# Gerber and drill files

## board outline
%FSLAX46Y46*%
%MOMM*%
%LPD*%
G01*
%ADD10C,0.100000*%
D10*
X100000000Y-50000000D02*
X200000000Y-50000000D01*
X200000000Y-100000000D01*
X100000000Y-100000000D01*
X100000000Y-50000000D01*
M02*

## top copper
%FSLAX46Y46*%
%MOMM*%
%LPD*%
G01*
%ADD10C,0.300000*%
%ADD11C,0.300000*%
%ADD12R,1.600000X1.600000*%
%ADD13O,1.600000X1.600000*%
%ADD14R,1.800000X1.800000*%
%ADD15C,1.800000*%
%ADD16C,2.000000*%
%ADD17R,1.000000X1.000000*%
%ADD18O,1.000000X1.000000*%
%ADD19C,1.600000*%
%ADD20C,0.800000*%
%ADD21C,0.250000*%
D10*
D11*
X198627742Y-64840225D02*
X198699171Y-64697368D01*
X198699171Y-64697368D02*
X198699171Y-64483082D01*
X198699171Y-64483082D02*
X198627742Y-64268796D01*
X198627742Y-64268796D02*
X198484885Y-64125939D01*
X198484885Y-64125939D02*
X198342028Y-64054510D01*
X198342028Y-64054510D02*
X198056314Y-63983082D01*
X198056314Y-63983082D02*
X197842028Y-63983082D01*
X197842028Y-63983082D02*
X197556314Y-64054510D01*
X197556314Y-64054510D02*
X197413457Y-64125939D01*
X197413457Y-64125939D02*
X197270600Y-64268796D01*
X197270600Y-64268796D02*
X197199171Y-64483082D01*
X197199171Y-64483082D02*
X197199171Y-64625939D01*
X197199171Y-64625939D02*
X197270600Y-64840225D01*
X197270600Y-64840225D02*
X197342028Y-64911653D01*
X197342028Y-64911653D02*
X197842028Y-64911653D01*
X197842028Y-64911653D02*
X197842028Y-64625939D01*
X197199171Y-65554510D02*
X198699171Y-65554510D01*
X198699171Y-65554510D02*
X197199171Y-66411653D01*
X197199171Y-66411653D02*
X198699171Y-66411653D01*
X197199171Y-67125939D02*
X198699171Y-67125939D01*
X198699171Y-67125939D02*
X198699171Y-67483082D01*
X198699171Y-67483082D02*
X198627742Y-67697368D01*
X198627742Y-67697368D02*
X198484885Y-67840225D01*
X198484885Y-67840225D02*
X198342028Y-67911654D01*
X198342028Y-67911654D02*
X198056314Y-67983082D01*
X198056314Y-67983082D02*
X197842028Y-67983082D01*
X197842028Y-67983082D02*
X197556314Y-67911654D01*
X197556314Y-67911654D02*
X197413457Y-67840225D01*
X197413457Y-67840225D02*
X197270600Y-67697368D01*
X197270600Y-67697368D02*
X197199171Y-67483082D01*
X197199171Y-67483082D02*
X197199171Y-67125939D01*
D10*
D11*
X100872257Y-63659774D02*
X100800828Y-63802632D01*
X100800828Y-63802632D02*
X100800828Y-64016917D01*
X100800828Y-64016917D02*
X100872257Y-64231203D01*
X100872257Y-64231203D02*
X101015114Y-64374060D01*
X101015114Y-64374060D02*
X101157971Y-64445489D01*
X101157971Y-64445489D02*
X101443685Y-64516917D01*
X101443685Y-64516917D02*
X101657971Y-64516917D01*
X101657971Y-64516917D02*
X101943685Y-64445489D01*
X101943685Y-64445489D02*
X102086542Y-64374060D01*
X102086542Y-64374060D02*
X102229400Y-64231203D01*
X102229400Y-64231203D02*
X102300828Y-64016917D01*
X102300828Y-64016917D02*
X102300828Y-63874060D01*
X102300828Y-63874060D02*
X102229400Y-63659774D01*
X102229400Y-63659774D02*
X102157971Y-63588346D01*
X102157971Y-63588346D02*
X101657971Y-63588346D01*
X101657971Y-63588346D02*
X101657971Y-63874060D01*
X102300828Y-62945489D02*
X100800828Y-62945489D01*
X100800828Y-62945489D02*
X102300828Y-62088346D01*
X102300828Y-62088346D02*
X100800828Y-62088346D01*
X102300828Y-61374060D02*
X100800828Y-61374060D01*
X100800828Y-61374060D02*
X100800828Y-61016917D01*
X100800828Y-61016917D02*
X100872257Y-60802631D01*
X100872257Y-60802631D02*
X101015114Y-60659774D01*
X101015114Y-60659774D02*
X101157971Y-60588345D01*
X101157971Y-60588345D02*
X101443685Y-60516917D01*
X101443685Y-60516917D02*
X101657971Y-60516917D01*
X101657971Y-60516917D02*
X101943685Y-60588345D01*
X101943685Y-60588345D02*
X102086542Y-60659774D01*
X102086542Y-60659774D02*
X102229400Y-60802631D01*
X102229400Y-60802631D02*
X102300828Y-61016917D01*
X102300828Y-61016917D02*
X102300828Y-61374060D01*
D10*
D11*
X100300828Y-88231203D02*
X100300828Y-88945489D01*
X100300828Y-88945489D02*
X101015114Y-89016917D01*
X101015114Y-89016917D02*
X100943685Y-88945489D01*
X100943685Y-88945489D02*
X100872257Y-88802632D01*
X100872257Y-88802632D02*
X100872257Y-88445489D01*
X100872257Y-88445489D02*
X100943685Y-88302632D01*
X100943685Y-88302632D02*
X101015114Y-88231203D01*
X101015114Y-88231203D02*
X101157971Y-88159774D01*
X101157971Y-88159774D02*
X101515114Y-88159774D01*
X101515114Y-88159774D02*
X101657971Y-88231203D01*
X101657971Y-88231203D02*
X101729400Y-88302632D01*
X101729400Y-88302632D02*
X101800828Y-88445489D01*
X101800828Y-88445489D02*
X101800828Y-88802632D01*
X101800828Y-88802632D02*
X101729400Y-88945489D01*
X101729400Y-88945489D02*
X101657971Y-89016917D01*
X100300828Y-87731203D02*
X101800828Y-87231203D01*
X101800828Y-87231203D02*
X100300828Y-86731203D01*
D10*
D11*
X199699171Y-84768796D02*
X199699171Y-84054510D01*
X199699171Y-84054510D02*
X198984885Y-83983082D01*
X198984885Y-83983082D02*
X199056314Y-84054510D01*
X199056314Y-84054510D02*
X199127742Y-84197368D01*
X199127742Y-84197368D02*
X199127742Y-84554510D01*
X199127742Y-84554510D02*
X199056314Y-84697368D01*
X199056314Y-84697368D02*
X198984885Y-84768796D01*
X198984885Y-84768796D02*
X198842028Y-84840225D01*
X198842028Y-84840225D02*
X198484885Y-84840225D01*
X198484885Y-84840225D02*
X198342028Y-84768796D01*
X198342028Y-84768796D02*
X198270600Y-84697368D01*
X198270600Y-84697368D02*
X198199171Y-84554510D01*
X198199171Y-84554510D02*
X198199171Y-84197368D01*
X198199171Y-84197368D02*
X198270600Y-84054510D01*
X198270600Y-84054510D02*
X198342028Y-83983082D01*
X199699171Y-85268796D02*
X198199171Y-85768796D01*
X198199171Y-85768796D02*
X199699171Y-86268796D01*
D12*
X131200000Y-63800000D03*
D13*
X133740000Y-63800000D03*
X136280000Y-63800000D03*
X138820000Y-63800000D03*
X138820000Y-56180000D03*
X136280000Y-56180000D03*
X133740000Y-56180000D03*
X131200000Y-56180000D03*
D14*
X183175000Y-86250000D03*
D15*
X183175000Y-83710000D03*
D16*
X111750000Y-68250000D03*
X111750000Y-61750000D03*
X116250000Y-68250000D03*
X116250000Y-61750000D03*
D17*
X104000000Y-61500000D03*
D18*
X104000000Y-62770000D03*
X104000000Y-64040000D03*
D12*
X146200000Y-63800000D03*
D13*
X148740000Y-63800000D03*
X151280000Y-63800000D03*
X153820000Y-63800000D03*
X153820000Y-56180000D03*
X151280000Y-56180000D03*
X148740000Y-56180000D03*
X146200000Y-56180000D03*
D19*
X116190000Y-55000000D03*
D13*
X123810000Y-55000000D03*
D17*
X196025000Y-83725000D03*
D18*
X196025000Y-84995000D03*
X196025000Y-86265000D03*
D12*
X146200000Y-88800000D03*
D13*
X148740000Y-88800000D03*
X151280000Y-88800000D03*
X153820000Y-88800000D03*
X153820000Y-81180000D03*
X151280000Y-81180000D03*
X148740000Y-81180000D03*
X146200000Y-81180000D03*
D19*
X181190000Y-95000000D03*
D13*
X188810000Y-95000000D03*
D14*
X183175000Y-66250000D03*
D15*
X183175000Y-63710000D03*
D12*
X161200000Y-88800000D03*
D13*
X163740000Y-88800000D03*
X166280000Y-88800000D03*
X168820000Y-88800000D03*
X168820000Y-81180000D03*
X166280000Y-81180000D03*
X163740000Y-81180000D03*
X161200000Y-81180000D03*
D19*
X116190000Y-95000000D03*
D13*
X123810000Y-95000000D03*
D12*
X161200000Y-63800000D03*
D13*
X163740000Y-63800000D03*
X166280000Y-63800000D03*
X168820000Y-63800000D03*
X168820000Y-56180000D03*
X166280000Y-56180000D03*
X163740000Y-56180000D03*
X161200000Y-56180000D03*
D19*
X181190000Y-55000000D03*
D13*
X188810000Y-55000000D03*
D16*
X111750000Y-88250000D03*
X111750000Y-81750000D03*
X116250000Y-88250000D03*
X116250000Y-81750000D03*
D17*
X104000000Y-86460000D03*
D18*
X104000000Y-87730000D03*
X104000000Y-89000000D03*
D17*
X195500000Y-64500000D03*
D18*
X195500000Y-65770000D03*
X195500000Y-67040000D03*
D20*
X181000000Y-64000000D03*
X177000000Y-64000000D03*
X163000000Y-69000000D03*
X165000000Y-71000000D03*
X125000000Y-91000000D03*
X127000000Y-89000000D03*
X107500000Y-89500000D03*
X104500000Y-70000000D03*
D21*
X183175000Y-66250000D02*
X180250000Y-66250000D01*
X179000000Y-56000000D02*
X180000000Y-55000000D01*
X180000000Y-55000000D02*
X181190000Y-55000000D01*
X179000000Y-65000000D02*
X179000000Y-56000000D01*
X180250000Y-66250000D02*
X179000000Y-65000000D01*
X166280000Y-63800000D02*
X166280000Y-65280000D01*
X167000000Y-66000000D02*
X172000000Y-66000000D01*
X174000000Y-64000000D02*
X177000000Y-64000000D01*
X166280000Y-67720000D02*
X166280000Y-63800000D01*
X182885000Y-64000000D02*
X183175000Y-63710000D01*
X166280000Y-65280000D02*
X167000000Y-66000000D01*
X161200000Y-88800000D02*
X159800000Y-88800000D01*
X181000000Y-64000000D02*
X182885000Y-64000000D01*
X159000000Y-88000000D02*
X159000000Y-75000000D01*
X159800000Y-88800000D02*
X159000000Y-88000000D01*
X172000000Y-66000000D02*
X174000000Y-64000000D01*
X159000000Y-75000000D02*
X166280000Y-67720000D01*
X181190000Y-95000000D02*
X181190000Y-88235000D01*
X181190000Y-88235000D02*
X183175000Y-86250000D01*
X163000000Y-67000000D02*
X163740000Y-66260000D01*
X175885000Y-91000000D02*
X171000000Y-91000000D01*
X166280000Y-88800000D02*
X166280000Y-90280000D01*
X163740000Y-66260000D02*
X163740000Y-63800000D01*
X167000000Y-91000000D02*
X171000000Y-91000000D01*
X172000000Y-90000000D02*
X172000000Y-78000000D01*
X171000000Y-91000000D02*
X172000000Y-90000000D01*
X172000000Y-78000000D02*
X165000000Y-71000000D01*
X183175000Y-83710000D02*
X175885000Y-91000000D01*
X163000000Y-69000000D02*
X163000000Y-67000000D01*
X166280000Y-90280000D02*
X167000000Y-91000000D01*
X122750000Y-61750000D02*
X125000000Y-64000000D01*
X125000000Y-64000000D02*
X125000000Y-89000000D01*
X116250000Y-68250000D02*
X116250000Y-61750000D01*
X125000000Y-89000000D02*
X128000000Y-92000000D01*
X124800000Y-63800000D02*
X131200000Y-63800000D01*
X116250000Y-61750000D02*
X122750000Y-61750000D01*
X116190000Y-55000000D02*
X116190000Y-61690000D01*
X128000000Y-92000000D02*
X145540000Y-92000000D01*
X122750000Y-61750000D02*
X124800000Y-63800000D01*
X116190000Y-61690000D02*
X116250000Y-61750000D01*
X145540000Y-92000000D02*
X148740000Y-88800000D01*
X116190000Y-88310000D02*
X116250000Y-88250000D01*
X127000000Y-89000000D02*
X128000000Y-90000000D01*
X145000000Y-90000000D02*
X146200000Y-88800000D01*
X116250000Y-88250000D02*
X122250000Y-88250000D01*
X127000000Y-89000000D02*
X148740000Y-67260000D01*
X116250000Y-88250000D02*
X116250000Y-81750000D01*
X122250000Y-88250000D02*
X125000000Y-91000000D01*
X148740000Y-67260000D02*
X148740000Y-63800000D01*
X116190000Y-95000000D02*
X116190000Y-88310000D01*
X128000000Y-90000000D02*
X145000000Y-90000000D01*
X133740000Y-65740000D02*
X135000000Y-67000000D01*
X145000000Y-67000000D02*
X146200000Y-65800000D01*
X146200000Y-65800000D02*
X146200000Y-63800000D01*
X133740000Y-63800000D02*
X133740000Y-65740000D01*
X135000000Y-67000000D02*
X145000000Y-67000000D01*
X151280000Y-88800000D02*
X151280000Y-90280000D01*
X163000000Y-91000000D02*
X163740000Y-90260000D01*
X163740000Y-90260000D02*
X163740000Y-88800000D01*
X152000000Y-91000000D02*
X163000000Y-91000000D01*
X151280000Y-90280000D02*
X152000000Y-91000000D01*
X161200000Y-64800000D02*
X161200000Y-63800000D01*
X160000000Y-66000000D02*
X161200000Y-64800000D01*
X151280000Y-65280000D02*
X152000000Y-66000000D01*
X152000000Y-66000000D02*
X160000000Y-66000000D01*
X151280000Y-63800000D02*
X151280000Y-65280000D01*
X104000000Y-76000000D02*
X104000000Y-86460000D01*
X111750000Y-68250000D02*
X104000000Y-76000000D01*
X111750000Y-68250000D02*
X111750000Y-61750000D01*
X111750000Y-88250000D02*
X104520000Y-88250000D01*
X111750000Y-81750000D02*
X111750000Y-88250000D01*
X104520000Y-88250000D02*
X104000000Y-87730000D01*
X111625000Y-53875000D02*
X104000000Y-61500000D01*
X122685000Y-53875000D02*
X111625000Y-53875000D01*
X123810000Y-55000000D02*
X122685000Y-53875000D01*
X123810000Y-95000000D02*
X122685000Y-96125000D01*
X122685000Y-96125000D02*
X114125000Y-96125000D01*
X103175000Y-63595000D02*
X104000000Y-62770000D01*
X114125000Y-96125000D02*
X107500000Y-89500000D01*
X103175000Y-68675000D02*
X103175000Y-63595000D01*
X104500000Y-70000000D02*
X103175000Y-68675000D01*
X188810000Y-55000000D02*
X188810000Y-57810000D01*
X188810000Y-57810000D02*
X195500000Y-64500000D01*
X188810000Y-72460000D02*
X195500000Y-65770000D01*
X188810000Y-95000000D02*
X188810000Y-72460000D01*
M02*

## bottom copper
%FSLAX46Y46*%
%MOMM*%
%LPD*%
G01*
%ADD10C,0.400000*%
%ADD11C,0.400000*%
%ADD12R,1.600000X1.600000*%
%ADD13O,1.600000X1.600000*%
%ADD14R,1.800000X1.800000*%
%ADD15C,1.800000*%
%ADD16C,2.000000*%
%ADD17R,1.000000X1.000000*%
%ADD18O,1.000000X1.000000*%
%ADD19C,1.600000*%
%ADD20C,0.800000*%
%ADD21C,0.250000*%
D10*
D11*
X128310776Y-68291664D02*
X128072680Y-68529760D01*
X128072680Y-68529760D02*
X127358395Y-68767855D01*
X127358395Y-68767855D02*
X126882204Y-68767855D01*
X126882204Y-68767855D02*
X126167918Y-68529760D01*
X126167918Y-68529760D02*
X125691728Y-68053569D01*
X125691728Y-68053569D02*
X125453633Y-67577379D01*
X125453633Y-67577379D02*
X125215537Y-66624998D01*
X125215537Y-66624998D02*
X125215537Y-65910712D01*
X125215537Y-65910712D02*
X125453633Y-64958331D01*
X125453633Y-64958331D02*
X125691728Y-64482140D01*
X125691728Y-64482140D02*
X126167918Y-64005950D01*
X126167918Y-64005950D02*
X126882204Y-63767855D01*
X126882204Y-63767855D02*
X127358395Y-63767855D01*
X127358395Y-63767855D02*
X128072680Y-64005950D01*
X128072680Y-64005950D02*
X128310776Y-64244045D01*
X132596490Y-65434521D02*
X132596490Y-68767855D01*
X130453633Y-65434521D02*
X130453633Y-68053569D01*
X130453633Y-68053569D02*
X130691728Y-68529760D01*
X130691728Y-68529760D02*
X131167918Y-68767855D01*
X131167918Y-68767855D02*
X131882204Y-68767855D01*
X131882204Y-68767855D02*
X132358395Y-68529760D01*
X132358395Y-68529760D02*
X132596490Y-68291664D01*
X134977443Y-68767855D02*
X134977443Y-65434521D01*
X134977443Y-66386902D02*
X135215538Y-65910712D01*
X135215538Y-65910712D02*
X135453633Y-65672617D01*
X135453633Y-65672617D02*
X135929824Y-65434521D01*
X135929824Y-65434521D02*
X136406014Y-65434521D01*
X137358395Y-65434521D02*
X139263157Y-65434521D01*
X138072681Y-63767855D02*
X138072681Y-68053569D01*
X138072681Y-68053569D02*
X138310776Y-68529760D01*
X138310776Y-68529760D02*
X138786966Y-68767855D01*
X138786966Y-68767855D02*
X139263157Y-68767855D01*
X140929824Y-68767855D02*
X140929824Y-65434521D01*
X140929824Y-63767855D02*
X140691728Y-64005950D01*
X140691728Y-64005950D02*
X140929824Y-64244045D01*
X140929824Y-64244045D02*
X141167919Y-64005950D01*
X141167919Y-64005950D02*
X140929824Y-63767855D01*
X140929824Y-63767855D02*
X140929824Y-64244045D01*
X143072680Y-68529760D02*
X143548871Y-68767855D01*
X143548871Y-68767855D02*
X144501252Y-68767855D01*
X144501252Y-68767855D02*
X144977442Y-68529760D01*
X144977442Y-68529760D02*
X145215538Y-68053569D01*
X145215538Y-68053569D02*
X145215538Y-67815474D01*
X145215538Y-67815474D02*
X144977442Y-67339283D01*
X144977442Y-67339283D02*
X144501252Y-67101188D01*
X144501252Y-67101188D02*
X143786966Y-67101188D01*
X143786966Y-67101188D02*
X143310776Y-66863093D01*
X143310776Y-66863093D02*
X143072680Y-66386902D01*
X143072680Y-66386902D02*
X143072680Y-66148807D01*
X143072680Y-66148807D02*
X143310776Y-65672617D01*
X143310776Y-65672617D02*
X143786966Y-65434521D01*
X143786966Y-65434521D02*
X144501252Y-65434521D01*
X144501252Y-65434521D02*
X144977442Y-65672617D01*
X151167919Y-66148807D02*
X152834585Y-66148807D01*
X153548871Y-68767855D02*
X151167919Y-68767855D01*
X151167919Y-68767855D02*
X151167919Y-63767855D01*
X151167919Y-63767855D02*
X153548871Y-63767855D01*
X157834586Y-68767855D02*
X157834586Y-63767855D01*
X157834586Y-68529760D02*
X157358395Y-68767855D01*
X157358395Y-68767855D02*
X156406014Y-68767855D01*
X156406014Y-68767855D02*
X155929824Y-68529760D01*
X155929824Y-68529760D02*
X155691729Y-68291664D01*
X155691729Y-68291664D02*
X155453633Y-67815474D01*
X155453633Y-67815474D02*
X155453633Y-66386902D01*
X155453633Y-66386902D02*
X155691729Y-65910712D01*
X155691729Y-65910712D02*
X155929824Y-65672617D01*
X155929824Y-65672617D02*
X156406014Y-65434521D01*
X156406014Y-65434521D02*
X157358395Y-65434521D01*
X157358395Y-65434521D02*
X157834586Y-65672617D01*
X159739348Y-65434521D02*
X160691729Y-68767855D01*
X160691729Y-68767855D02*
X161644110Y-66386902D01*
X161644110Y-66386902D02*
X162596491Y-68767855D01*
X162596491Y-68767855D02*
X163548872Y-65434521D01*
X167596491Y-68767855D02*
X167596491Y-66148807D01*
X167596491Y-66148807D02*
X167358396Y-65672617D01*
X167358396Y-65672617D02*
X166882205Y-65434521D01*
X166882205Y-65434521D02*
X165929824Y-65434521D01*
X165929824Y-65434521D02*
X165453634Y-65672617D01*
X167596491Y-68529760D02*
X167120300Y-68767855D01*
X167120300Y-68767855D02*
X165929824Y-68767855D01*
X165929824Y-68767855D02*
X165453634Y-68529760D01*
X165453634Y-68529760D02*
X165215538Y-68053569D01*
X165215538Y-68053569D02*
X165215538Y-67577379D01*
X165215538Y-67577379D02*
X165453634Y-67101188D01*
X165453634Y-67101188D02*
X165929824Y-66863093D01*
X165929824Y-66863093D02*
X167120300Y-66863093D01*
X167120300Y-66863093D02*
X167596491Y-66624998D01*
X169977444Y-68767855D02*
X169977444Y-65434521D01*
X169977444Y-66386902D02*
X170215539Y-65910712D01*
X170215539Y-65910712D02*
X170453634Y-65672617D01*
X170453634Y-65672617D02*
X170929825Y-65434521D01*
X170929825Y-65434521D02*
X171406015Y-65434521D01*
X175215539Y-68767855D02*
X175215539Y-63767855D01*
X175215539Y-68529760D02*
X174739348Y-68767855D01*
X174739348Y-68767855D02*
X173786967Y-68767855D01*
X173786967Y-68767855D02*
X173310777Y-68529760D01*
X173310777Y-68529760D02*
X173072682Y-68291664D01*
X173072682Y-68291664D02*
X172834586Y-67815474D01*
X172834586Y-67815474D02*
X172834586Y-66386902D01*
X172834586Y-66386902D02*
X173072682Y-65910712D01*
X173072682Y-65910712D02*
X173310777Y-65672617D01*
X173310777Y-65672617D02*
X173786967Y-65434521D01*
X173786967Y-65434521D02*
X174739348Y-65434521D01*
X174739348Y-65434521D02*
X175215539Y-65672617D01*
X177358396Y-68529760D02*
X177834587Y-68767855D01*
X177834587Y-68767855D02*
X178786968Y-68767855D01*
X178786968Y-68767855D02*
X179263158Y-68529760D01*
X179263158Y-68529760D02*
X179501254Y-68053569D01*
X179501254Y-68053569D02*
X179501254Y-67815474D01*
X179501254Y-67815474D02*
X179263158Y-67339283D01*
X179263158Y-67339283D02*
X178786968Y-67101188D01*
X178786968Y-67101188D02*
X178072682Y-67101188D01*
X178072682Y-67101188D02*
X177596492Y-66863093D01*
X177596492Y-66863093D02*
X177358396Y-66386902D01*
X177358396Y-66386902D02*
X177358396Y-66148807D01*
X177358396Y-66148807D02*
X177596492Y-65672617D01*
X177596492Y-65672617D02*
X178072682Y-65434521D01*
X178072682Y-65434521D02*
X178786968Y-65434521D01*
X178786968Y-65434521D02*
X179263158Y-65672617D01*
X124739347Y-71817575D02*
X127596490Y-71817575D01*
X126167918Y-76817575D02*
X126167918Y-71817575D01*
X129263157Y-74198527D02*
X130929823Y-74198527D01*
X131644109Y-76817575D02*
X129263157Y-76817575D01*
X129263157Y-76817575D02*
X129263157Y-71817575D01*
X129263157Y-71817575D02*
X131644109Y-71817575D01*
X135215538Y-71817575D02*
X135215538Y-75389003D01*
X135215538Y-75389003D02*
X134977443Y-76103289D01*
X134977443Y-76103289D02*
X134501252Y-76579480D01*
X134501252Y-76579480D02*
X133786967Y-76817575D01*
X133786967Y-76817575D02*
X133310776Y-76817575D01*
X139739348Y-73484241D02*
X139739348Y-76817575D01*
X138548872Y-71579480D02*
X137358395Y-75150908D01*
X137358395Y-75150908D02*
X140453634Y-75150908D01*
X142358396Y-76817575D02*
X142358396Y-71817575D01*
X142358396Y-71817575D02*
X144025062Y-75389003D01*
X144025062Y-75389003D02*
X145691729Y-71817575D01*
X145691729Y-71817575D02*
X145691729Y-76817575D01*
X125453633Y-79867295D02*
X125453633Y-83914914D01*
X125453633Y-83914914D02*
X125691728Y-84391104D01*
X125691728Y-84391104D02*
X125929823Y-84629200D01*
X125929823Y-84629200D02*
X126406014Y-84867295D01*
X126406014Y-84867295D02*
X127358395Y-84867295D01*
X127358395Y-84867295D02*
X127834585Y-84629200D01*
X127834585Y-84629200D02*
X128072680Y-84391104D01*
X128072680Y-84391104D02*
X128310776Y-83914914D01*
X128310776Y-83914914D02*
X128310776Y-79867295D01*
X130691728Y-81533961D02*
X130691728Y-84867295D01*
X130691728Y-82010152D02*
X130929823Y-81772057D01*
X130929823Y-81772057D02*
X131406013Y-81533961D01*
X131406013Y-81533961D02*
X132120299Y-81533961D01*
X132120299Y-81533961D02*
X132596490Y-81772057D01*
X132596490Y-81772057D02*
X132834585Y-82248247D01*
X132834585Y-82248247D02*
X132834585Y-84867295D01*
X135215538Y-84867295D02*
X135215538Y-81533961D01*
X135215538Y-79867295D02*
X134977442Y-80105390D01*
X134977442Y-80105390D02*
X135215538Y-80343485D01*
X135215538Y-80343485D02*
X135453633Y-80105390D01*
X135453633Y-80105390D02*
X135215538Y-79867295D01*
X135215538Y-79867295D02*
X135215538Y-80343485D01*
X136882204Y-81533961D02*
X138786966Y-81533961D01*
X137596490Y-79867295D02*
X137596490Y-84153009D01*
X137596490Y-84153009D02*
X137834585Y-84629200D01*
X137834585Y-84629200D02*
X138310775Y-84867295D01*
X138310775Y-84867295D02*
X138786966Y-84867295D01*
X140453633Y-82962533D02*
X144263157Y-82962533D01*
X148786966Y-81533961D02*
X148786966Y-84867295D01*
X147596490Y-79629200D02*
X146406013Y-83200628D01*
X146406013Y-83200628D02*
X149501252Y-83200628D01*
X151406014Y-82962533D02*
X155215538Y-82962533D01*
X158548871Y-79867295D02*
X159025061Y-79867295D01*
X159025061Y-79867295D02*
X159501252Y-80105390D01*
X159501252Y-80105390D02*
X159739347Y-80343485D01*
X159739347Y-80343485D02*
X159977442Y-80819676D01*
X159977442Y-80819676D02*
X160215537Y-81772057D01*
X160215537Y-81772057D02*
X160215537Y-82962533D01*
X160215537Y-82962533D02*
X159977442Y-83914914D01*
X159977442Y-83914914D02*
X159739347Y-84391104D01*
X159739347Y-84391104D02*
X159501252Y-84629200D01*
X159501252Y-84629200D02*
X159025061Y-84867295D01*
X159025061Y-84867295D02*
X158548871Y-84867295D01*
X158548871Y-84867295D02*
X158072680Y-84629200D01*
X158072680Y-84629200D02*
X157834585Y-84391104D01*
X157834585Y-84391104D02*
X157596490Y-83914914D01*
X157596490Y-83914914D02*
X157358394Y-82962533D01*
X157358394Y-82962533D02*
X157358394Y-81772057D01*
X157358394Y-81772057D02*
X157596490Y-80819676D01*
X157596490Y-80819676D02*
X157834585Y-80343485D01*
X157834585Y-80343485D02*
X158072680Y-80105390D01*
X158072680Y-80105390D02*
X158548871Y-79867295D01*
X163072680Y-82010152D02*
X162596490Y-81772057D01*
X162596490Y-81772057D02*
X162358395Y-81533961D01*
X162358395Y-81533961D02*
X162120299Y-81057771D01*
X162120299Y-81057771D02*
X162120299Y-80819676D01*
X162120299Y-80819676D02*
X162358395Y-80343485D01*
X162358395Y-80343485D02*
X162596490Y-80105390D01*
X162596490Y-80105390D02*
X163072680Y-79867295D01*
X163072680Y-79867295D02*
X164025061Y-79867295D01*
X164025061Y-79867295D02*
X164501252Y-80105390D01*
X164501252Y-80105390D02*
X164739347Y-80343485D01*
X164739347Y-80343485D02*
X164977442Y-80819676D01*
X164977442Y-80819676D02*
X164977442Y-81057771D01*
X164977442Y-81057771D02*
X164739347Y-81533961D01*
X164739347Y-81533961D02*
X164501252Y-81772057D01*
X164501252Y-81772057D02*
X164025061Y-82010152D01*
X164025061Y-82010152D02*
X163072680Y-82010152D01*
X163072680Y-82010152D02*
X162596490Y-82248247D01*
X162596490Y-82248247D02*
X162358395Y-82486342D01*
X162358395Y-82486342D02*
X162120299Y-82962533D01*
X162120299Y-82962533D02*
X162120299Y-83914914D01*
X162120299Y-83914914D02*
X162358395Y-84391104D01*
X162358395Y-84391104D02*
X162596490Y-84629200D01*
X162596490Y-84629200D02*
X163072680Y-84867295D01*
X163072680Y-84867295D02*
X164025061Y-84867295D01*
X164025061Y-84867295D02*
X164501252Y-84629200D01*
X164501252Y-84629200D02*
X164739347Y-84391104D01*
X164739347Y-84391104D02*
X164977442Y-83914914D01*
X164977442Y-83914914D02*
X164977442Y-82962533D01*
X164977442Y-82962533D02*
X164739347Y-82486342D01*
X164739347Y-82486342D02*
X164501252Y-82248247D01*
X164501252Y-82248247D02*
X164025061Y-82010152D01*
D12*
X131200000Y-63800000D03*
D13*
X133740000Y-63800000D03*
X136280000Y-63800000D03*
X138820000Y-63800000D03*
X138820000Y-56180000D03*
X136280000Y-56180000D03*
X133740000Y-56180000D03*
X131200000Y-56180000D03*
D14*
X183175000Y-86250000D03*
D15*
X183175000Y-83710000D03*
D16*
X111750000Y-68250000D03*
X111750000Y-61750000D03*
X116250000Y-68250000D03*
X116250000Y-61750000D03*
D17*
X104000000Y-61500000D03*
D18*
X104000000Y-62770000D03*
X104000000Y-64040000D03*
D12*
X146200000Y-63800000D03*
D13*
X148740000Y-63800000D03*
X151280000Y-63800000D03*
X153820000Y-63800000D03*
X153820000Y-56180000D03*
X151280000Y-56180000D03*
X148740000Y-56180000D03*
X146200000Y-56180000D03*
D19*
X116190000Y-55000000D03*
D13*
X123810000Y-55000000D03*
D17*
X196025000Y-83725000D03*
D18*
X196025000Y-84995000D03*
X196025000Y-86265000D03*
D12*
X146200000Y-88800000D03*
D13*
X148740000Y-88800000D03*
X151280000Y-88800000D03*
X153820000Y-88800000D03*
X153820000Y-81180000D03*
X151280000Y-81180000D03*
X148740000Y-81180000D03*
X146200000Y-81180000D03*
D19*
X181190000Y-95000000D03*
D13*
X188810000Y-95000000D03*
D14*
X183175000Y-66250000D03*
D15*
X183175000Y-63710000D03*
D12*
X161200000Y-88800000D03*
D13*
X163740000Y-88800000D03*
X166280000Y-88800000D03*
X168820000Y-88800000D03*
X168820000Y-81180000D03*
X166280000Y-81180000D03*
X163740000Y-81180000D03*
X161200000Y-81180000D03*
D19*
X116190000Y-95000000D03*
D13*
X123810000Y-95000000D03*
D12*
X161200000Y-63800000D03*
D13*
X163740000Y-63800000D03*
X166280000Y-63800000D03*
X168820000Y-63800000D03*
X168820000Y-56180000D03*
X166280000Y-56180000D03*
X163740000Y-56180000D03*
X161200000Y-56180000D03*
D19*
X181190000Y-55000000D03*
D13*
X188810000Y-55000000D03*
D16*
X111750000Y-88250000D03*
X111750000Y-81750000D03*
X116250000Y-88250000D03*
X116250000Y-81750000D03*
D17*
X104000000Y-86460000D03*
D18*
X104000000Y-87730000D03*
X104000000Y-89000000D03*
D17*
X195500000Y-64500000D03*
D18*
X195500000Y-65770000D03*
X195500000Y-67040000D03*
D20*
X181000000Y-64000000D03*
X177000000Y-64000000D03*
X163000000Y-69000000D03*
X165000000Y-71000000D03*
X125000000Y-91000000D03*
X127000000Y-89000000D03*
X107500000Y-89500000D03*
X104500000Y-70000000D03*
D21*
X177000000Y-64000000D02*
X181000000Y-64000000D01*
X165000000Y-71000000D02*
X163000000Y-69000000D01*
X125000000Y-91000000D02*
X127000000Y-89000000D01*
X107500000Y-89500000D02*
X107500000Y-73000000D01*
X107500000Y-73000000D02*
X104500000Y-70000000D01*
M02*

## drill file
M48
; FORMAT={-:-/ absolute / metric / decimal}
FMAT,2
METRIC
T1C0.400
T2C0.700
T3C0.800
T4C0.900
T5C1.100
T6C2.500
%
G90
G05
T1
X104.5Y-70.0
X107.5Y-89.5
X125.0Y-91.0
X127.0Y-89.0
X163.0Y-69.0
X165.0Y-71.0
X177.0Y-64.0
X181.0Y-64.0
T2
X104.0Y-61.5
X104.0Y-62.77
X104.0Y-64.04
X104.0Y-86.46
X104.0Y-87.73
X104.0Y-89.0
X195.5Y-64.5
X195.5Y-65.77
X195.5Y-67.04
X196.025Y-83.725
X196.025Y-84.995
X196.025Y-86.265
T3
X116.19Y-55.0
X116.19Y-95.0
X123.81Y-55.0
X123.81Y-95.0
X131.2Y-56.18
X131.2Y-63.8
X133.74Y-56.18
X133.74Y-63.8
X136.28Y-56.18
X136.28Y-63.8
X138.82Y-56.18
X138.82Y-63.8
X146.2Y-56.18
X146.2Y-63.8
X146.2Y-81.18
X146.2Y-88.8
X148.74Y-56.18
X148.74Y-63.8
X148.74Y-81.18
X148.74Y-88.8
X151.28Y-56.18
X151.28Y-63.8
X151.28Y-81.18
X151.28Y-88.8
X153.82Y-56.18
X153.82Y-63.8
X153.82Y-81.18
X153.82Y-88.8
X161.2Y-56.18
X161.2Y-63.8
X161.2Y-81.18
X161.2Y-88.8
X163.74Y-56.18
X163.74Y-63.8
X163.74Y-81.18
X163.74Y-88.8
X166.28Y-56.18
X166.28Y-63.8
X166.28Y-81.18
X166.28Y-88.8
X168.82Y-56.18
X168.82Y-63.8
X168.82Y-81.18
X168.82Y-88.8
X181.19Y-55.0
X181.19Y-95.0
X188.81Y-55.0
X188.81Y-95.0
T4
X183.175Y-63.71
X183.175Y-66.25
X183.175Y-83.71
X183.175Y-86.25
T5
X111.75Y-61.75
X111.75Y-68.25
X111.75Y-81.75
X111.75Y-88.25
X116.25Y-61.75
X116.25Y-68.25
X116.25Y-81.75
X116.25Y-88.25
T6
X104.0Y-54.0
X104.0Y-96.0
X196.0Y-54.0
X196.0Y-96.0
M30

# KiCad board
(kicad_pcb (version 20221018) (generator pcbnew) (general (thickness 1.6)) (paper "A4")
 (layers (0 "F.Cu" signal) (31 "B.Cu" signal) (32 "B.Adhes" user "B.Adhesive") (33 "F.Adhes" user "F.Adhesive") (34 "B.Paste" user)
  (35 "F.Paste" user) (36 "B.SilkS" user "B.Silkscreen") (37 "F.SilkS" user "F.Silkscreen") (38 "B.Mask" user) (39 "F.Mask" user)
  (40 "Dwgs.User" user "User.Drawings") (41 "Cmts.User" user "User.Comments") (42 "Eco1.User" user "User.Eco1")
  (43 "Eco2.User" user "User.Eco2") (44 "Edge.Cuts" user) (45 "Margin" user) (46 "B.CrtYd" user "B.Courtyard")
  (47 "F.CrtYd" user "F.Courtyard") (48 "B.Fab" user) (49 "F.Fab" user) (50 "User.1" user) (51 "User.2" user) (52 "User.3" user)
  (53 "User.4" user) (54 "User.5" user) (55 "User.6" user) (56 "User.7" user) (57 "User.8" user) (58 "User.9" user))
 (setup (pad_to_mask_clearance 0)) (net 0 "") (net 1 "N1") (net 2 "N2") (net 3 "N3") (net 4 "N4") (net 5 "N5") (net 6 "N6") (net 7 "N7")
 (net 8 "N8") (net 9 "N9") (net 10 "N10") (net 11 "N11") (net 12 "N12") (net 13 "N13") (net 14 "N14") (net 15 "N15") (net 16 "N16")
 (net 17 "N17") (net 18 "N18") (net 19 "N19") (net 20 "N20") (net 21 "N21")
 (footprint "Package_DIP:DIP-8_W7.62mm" (layer "F.Cu") (at 131.2 63.8 90)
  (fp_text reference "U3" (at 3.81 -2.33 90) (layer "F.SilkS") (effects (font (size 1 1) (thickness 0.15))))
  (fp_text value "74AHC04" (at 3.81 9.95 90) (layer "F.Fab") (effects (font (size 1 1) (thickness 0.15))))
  (pad "1" thru_hole rect (at 0 0 90) (size 1.6 1.6) (drill 0.8) (layers "*.Cu" "*.Mask") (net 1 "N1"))
  (pad "2" thru_hole oval (at 0 2.54 90) (size 1.6 1.6) (drill 0.8) (layers "*.Cu" "*.Mask") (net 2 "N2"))
  (pad "3" thru_hole oval (at 0 5.08 90) (size 1.6 1.6) (drill 0.8) (layers "*.Cu" "*.Mask"))
  (pad "4" thru_hole oval (at 0 7.62 90) (size 1.6 1.6) (drill 0.8) (layers "*.Cu" "*.Mask"))
  (pad "5" thru_hole oval (at 7.62 7.62 90) (size 1.6 1.6) (drill 0.8) (layers "*.Cu" "*.Mask"))
  (pad "6" thru_hole oval (at 7.62 5.08 90) (size 1.6 1.6) (drill 0.8) (layers "*.Cu" "*.Mask"))
  (pad "7" thru_hole oval (at 7.62 2.54 90) (size 1.6 1.6) (drill 0.8) (layers "*.Cu" "*.Mask"))
  (pad "8" thru_hole oval (at 7.62 0 90) (size 1.6 1.6) (drill 0.8) (layers "*.Cu" "*.Mask")))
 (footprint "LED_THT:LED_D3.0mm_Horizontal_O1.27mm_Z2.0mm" (layer "F.Cu") (at 183.175 86.25 90)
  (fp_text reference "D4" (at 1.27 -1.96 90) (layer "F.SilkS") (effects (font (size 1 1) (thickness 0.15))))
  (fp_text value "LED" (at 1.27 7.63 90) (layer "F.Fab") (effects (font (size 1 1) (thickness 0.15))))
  (pad "1" thru_hole rect (at 0 0 90) (size 1.8 1.8) (drill 0.9) (layers "*.Cu" "*.Mask") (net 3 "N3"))
  (pad "2" thru_hole circle (at 2.54 0 90) (size 1.8 1.8) (drill 0.9) (layers "*.Cu" "*.Mask") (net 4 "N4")))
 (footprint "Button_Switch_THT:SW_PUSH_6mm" (layer "F.Cu") (at 111.75 68.25 90)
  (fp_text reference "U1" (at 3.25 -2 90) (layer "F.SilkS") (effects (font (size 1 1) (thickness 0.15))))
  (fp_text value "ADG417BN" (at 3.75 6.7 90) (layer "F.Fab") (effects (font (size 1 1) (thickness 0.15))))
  (pad "1" thru_hole circle (at 0 0 180) (size 2 2) (drill 1.1) (layers "*.Cu" "*.Mask") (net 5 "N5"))
  (pad "1" thru_hole circle (at 6.5 0 180) (size 2 2) (drill 1.1) (layers "*.Cu" "*.Mask") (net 5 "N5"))
  (pad "2" thru_hole circle (at 0 4.5 180) (size 2 2) (drill 1.1) (layers "*.Cu" "*.Mask") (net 1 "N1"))
  (pad "2" thru_hole circle (at 6.5 4.5 180) (size 2 2) (drill 1.1) (layers "*.Cu" "*.Mask") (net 1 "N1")))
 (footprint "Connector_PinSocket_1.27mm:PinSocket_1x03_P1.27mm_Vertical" (layer "F.Cu") (at 104 61.5)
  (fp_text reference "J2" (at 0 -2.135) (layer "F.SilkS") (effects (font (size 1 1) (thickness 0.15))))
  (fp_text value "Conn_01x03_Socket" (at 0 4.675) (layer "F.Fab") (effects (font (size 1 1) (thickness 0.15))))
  (pad "1" thru_hole rect (at 0 0) (size 1 1) (drill 0.7) (layers "*.Cu" "*.Mask") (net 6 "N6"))
  (pad "2" thru_hole oval (at 0 1.27) (size 1 1) (drill 0.7) (layers "*.Cu" "*.Mask") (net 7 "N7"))
  (pad "3" thru_hole oval (at 0 2.54) (size 1 1) (drill 0.7) (layers "*.Cu" "*.Mask") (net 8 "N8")))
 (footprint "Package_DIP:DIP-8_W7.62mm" (layer "F.Cu") (at 146.2 63.8 90)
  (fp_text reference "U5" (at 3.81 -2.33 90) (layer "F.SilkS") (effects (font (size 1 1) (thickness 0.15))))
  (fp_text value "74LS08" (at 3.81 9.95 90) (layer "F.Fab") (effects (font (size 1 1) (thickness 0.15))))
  (pad "1" thru_hole rect (at 0 0 90) (size 1.6 1.6) (drill 0.8) (layers "*.Cu" "*.Mask") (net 2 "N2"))
  (pad "2" thru_hole oval (at 0 2.54 90) (size 1.6 1.6) (drill 0.8) (layers "*.Cu" "*.Mask") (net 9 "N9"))
  (pad "3" thru_hole oval (at 0 5.08 90) (size 1.6 1.6) (drill 0.8) (layers "*.Cu" "*.Mask") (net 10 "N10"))
  (pad "4" thru_hole oval (at 0 7.62 90) (size 1.6 1.6) (drill 0.8) (layers "*.Cu" "*.Mask"))
  (pad "5" thru_hole oval (at 7.62 7.62 90) (size 1.6 1.6) (drill 0.8) (layers "*.Cu" "*.Mask"))
  (pad "6" thru_hole oval (at 7.62 5.08 90) (size 1.6 1.6) (drill 0.8) (layers "*.Cu" "*.Mask"))
  (pad "7" thru_hole oval (at 7.62 2.54 90) (size 1.6 1.6) (drill 0.8) (layers "*.Cu" "*.Mask"))
  (pad "8" thru_hole oval (at 7.62 0 90) (size 1.6 1.6) (drill 0.8) (layers "*.Cu" "*.Mask")))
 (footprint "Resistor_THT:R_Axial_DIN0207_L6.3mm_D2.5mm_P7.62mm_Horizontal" (layer "F.Cu") (at 116.19 55)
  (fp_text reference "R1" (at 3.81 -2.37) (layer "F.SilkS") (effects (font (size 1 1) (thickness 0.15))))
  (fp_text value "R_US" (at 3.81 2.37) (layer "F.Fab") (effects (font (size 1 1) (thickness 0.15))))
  (pad "1" thru_hole circle (at 0 0) (size 1.6 1.6) (drill 0.8) (layers "*.Cu" "*.Mask") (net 1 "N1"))
  (pad "2" thru_hole oval (at 7.62 0) (size 1.6 1.6) (drill 0.8) (layers "*.Cu" "*.Mask") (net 6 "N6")))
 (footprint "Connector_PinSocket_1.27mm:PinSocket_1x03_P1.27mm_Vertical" (layer "F.Cu") (at 196.025 83.725)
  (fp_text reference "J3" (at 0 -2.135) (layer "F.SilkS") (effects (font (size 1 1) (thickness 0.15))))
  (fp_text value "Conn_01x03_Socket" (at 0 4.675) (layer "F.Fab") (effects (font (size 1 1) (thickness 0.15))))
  (pad "1" thru_hole rect (at 0 0) (size 1 1) (drill 0.7) (layers "*.Cu" "*.Mask") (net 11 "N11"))
  (pad "2" thru_hole oval (at 0 1.27) (size 1 1) (drill 0.7) (layers "*.Cu" "*.Mask") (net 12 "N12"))
  (pad "3" thru_hole oval (at 0 2.54) (size 1 1) (drill 0.7) (layers "*.Cu" "*.Mask") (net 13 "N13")))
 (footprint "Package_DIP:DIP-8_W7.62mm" (layer "F.Cu") (at 146.2 88.8 90)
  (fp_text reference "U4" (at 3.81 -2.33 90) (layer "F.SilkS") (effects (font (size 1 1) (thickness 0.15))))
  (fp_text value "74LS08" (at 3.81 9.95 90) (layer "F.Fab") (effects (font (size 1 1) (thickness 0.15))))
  (pad "1" thru_hole rect (at 0 0 90) (size 1.6 1.6) (drill 0.8) (layers "*.Cu" "*.Mask") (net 9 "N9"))
  (pad "2" thru_hole oval (at 0 2.54 90) (size 1.6 1.6) (drill 0.8) (layers "*.Cu" "*.Mask") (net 1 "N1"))
  (pad "3" thru_hole oval (at 0 5.08 90) (size 1.6 1.6) (drill 0.8) (layers "*.Cu" "*.Mask") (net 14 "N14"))
  (pad "4" thru_hole oval (at 0 7.62 90) (size 1.6 1.6) (drill 0.8) (layers "*.Cu" "*.Mask"))
  (pad "5" thru_hole oval (at 7.62 7.62 90) (size 1.6 1.6) (drill 0.8) (layers "*.Cu" "*.Mask"))
  (pad "6" thru_hole oval (at 7.62 5.08 90) (size 1.6 1.6) (drill 0.8) (layers "*.Cu" "*.Mask"))
  (pad "7" thru_hole oval (at 7.62 2.54 90) (size 1.6 1.6) (drill 0.8) (layers "*.Cu" "*.Mask"))
  (pad "8" thru_hole oval (at 7.62 0 90) (size 1.6 1.6) (drill 0.8) (layers "*.Cu" "*.Mask")))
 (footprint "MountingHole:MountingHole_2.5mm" (layer "F.Cu") (at 196 96)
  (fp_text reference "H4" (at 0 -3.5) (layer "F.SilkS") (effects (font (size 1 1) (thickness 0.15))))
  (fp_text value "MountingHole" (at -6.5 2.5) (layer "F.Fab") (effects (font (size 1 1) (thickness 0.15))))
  (pad "" np_thru_hole circle (at 0 0) (size 2.5 2.5) (drill 2.5) (layers "*.Cu" "*.Mask")))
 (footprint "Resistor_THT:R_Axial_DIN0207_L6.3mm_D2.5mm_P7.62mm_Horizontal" (layer "F.Cu") (at 181.19 95)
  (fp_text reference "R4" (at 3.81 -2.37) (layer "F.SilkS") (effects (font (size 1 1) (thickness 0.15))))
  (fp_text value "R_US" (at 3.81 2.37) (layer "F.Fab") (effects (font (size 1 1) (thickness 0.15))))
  (pad "1" thru_hole circle (at 0 0) (size 1.6 1.6) (drill 0.8) (layers "*.Cu" "*.Mask") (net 3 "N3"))
  (pad "2" thru_hole oval (at 7.62 0) (size 1.6 1.6) (drill 0.8) (layers "*.Cu" "*.Mask") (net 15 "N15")))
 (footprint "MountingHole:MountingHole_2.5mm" (layer "F.Cu") (at 104 54)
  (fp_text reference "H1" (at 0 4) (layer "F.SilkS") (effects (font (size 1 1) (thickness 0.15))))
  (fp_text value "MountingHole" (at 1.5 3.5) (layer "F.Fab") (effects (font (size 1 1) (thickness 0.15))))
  (pad "" np_thru_hole circle (at 0 0) (size 2.5 2.5) (drill 2.5) (layers "*.Cu" "*.Mask")))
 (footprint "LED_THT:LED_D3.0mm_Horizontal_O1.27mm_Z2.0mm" (layer "F.Cu") (at 183.175 66.25 90)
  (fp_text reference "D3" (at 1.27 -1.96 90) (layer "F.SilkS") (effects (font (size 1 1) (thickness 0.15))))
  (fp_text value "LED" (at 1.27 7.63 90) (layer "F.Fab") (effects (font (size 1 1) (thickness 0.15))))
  (pad "1" thru_hole rect (at 0 0 90) (size 1.8 1.8) (drill 0.9) (layers "*.Cu" "*.Mask") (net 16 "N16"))
  (pad "2" thru_hole circle (at 2.54 0 90) (size 1.8 1.8) (drill 0.9) (layers "*.Cu" "*.Mask") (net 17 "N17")))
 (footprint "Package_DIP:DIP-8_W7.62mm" (layer "F.Cu") (at 161.2 88.8 90)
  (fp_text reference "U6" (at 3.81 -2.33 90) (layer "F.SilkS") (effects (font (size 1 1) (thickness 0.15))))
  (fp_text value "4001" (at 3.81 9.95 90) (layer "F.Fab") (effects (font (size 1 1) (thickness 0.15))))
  (pad "1" thru_hole rect (at 0 0 90) (size 1.6 1.6) (drill 0.8) (layers "*.Cu" "*.Mask") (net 17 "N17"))
  (pad "2" thru_hole oval (at 0 2.54 90) (size 1.6 1.6) (drill 0.8) (layers "*.Cu" "*.Mask") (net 14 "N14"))
  (pad "3" thru_hole oval (at 0 5.08 90) (size 1.6 1.6) (drill 0.8) (layers "*.Cu" "*.Mask") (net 4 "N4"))
  (pad "4" thru_hole oval (at 0 7.62 90) (size 1.6 1.6) (drill 0.8) (layers "*.Cu" "*.Mask"))
  (pad "5" thru_hole oval (at 7.62 7.62 90) (size 1.6 1.6) (drill 0.8) (layers "*.Cu" "*.Mask"))
  (pad "6" thru_hole oval (at 7.62 5.08 90) (size 1.6 1.6) (drill 0.8) (layers "*.Cu" "*.Mask"))
  (pad "7" thru_hole oval (at 7.62 2.54 90) (size 1.6 1.6) (drill 0.8) (layers "*.Cu" "*.Mask"))
  (pad "8" thru_hole oval (at 7.62 0 90) (size 1.6 1.6) (drill 0.8) (layers "*.Cu" "*.Mask")))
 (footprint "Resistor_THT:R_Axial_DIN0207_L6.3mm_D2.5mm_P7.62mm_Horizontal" (layer "F.Cu") (at 116.19 95)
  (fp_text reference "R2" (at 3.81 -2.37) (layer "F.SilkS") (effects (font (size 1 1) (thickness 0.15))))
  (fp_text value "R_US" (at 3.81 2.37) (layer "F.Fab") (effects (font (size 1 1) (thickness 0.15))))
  (pad "1" thru_hole circle (at 0 0) (size 1.6 1.6) (drill 0.8) (layers "*.Cu" "*.Mask") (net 9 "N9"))
  (pad "2" thru_hole oval (at 7.62 0) (size 1.6 1.6) (drill 0.8) (layers "*.Cu" "*.Mask") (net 7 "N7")))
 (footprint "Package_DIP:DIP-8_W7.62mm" (layer "F.Cu") (at 161.2 63.8 90)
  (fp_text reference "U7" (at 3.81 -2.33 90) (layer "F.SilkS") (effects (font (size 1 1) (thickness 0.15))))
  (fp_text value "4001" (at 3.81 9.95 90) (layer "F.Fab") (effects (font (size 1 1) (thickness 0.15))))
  (pad "1" thru_hole rect (at 0 0 90) (size 1.6 1.6) (drill 0.8) (layers "*.Cu" "*.Mask") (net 10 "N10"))
  (pad "2" thru_hole oval (at 0 2.54 90) (size 1.6 1.6) (drill 0.8) (layers "*.Cu" "*.Mask") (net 4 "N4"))
  (pad "3" thru_hole oval (at 0 5.08 90) (size 1.6 1.6) (drill 0.8) (layers "*.Cu" "*.Mask") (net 17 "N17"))
  (pad "4" thru_hole oval (at 0 7.62 90) (size 1.6 1.6) (drill 0.8) (layers "*.Cu" "*.Mask"))
  (pad "5" thru_hole oval (at 7.62 7.62 90) (size 1.6 1.6) (drill 0.8) (layers "*.Cu" "*.Mask"))
  (pad "6" thru_hole oval (at 7.62 5.08 90) (size 1.6 1.6) (drill 0.8) (layers "*.Cu" "*.Mask"))
  (pad "7" thru_hole oval (at 7.62 2.54 90) (size 1.6 1.6) (drill 0.8) (layers "*.Cu" "*.Mask"))
  (pad "8" thru_hole oval (at 7.62 0 90) (size 1.6 1.6) (drill 0.8) (layers "*.Cu" "*.Mask")))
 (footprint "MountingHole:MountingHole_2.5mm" (layer "F.Cu") (at 104 96)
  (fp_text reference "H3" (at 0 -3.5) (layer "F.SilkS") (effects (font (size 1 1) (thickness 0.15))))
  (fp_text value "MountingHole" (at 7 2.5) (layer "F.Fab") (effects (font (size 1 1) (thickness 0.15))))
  (pad "" np_thru_hole circle (at 0 0) (size 2.5 2.5) (drill 2.5) (layers "*.Cu" "*.Mask")))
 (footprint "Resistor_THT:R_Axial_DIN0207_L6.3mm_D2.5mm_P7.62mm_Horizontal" (layer "F.Cu") (at 181.19 55)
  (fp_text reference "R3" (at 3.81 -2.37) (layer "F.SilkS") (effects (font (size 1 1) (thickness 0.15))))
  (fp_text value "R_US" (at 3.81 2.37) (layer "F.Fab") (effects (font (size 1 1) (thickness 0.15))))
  (pad "1" thru_hole circle (at 0 0) (size 1.6 1.6) (drill 0.8) (layers "*.Cu" "*.Mask") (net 16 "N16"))
  (pad "2" thru_hole oval (at 7.62 0) (size 1.6 1.6) (drill 0.8) (layers "*.Cu" "*.Mask") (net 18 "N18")))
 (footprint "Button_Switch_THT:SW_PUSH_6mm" (layer "F.Cu") (at 111.75 88.25 90)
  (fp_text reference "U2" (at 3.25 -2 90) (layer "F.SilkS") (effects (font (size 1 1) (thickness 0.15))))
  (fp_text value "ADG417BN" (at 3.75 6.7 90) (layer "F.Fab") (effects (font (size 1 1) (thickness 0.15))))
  (pad "1" thru_hole circle (at 0 0 180) (size 2 2) (drill 1.1) (layers "*.Cu" "*.Mask") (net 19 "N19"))
  (pad "1" thru_hole circle (at 6.5 0 180) (size 2 2) (drill 1.1) (layers "*.Cu" "*.Mask") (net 19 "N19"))
  (pad "2" thru_hole circle (at 0 4.5 180) (size 2 2) (drill 1.1) (layers "*.Cu" "*.Mask") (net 9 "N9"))
  (pad "2" thru_hole circle (at 6.5 4.5 180) (size 2 2) (drill 1.1) (layers "*.Cu" "*.Mask") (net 9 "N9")))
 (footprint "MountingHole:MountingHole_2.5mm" (layer "F.Cu") (at 196 54)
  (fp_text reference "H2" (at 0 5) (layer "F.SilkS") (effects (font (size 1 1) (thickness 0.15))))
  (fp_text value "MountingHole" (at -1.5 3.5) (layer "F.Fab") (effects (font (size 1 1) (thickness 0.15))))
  (pad "" np_thru_hole circle (at 0 0) (size 2.5 2.5) (drill 2.5) (layers "*.Cu" "*.Mask")))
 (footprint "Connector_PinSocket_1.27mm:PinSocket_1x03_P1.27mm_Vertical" (layer "F.Cu") (at 104 86.46)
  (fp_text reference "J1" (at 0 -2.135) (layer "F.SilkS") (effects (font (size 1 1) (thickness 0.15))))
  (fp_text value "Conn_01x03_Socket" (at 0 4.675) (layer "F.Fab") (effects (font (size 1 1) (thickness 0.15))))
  (pad "1" thru_hole rect (at 0 0) (size 1 1) (drill 0.7) (layers "*.Cu" "*.Mask") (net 5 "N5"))
  (pad "2" thru_hole oval (at 0 1.27) (size 1 1) (drill 0.7) (layers "*.Cu" "*.Mask") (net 19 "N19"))
  (pad "3" thru_hole oval (at 0 2.54) (size 1 1) (drill 0.7) (layers "*.Cu" "*.Mask") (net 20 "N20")))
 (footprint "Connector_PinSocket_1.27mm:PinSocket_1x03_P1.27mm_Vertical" (layer "F.Cu") (at 195.5 64.5)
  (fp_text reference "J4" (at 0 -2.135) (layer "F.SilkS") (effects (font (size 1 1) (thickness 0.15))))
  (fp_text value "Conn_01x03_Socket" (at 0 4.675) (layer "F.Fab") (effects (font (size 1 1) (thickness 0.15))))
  (pad "1" thru_hole rect (at 0 0) (size 1 1) (drill 0.7) (layers "*.Cu" "*.Mask") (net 18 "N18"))
  (pad "2" thru_hole oval (at 0 1.27) (size 1 1) (drill 0.7) (layers "*.Cu" "*.Mask") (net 15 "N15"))
  (pad "3" thru_hole oval (at 0 2.54) (size 1 1) (drill 0.7) (layers "*.Cu" "*.Mask") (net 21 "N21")))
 (gr_rect (start 100 50) (end 200 100) (stroke (width 0.1) (type default)) (fill none) (layer "Edge.Cuts"))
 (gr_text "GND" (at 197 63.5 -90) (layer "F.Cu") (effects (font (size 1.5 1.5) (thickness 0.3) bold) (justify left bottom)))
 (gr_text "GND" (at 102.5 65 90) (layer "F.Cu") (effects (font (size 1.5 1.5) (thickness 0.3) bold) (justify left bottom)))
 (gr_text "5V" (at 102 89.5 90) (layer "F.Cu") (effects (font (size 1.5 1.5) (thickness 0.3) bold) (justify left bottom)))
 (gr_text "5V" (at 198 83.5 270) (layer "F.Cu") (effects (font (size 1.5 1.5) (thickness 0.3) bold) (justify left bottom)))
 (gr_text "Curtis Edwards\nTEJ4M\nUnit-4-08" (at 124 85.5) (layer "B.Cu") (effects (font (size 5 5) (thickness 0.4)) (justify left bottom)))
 (segment (start 183.175 66.25) (end 180.25 66.25) (width 0.25) (layer "F.Cu") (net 16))
 (segment (start 179 56) (end 180 55) (width 0.25) (layer "F.Cu") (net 16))
 (segment (start 180 55) (end 181.19 55) (width 0.25) (layer "F.Cu") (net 16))
 (segment (start 179 65) (end 179 56) (width 0.25) (layer "F.Cu") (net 16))
 (segment (start 180.25 66.25) (end 179 65) (width 0.25) (layer "F.Cu") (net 16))
 (segment (start 166.28 63.8) (end 166.28 65.28) (width 0.25) (layer "F.Cu") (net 17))
 (segment (start 167 66) (end 172 66) (width 0.25) (layer "F.Cu") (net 17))
 (segment (start 174 64) (end 177 64) (width 0.25) (layer "F.Cu") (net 17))
 (segment (start 166.28 67.72) (end 166.28 63.8) (width 0.25) (layer "F.Cu") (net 17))
 (segment (start 182.885 64) (end 183.175 63.71) (width 0.25) (layer "F.Cu") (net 17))
 (segment (start 166.28 65.28) (end 167 66) (width 0.25) (layer "F.Cu") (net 17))
 (segment (start 161.2 88.8) (end 159.8 88.8) (width 0.25) (layer "F.Cu") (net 17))
 (segment (start 181 64) (end 182.885 64) (width 0.25) (layer "F.Cu") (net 17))
 (segment (start 159 88) (end 159 75) (width 0.25) (layer "F.Cu") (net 17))
 (segment (start 159.8 88.8) (end 159 88) (width 0.25) (layer "F.Cu") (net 17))
 (segment (start 172 66) (end 174 64) (width 0.25) (layer "F.Cu") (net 17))
 (segment (start 159 75) (end 166.28 67.72) (width 0.25) (layer "F.Cu") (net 17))
 (via (at 181 64) (size 0.8) (drill 0.4) (layers "F.Cu" "B.Cu") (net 17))
 (via (at 177 64) (size 0.8) (drill 0.4) (layers "F.Cu" "B.Cu") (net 17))
 (segment (start 177 64) (end 181 64) (width 0.25) (layer "B.Cu") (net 17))
 (segment (start 181.19 95) (end 181.19 88.235) (width 0.25) (layer "F.Cu") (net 3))
 (segment (start 181.19 88.235) (end 183.175 86.25) (width 0.25) (layer "F.Cu") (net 3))
 (segment (start 163 67) (end 163.74 66.26) (width 0.25) (layer "F.Cu") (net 4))
 (segment (start 175.885 91) (end 171 91) (width 0.25) (layer "F.Cu") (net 4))
 (segment (start 166.28 88.8) (end 166.28 90.28) (width 0.25) (layer "F.Cu") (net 4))
 (segment (start 163.74 66.26) (end 163.74 63.8) (width 0.25) (layer "F.Cu") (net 4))
 (segment (start 167 91) (end 171 91) (width 0.25) (layer "F.Cu") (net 4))
 (segment (start 172 90) (end 172 78) (width 0.25) (layer "F.Cu") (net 4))
 (segment (start 171 91) (end 172 90) (width 0.25) (layer "F.Cu") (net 4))
 (segment (start 172 78) (end 165 71) (width 0.25) (layer "F.Cu") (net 4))
 (segment (start 183.175 83.71) (end 175.885 91) (width 0.25) (layer "F.Cu") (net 4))
 (segment (start 163 69) (end 163 67) (width 0.25) (layer "F.Cu") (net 4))
 (segment (start 166.28 90.28) (end 167 91) (width 0.25) (layer "F.Cu") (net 4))
 (via (at 163 69) (size 0.8) (drill 0.4) (layers "F.Cu" "B.Cu") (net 4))
 (via (at 165 71) (size 0.8) (drill 0.4) (layers "F.Cu" "B.Cu") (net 4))
 (segment (start 165 71) (end 163 69) (width 0.25) (layer "B.Cu") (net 4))
 (segment (start 122.75 61.75) (end 125 64) (width 0.25) (layer "F.Cu") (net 1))
 (segment (start 125 64) (end 125 89) (width 0.25) (layer "F.Cu") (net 1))
 (segment (start 116.25 68.25) (end 116.25 61.75) (width 0.25) (layer "F.Cu") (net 1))
 (segment (start 125 89) (end 128 92) (width 0.25) (layer "F.Cu") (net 1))
 (segment (start 124.8 63.8) (end 131.2 63.8) (width 0.25) (layer "F.Cu") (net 1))
 (segment (start 116.25 61.75) (end 122.75 61.75) (width 0.25) (layer "F.Cu") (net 1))
 (segment (start 116.19 55) (end 116.19 61.69) (width 0.25) (layer "F.Cu") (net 1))
 (segment (start 128 92) (end 145.54 92) (width 0.25) (layer "F.Cu") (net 1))
 (segment (start 122.75 61.75) (end 124.8 63.8) (width 0.25) (layer "F.Cu") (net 1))
 (segment (start 116.19 61.69) (end 116.25 61.75) (width 0.25) (layer "F.Cu") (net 1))
 (segment (start 145.54 92) (end 148.74 88.8) (width 0.25) (layer "F.Cu") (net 1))
 (segment (start 116.19 88.31) (end 116.25 88.25) (width 0.25) (layer "F.Cu") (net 9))
 (segment (start 127 89) (end 128 90) (width 0.25) (layer "F.Cu") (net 9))
 (segment (start 145 90) (end 146.2 88.8) (width 0.25) (layer "F.Cu") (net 9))
 (segment (start 116.25 88.25) (end 122.25 88.25) (width 0.25) (layer "F.Cu") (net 9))
 (segment (start 127 89) (end 148.74 67.26) (width 0.25) (layer "F.Cu") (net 9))
 (segment (start 116.25 88.25) (end 116.25 81.75) (width 0.25) (layer "F.Cu") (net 9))
 (segment (start 122.25 88.25) (end 125 91) (width 0.25) (layer "F.Cu") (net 9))
 (segment (start 148.74 67.26) (end 148.74 63.8) (width 0.25) (layer "F.Cu") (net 9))
 (segment (start 116.19 95) (end 116.19 88.31) (width 0.25) (layer "F.Cu") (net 9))
 (segment (start 128 90) (end 145 90) (width 0.25) (layer "F.Cu") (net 9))
 (via (at 125 91) (size 0.8) (drill 0.4) (layers "F.Cu" "B.Cu") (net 9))
 (via (at 127 89) (size 0.8) (drill 0.4) (layers "F.Cu" "B.Cu") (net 9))
 (segment (start 125 91) (end 127 89) (width 0.25) (layer "B.Cu") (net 9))
 (segment (start 133.74 65.74) (end 135 67) (width 0.25) (layer "F.Cu") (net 2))
 (segment (start 145 67) (end 146.2 65.8) (width 0.25) (layer "F.Cu") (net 2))
 (segment (start 146.2 65.8) (end 146.2 63.8) (width 0.25) (layer "F.Cu") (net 2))
 (segment (start 133.74 63.8) (end 133.74 65.74) (width 0.25) (layer "F.Cu") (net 2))
 (segment (start 135 67) (end 145 67) (width 0.25) (layer "F.Cu") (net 2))
 (segment (start 151.28 88.8) (end 151.28 90.28) (width 0.25) (layer "F.Cu") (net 14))
 (segment (start 163 91) (end 163.74 90.26) (width 0.25) (layer "F.Cu") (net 14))
 (segment (start 163.74 90.26) (end 163.74 88.8) (width 0.25) (layer "F.Cu") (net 14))
 (segment (start 152 91) (end 163 91) (width 0.25) (layer "F.Cu") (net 14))
 (segment (start 151.28 90.28) (end 152 91) (width 0.25) (layer "F.Cu") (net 14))
 (segment (start 161.2 64.8) (end 161.2 63.8) (width 0.25) (layer "F.Cu") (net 10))
 (segment (start 160 66) (end 161.2 64.8) (width 0.25) (layer "F.Cu") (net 10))
 (segment (start 151.28 65.28) (end 152 66) (width 0.25) (layer "F.Cu") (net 10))
 (segment (start 152 66) (end 160 66) (width 0.25) (layer "F.Cu") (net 10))
 (segment (start 151.28 63.8) (end 151.28 65.28) (width 0.25) (layer "F.Cu") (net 10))
 (segment (start 104 76) (end 104 86.46) (width 0.25) (layer "F.Cu") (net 5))
 (segment (start 111.75 68.25) (end 104 76) (width 0.25) (layer "F.Cu") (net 5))
 (segment (start 111.75 68.25) (end 111.75 61.75) (width 0.25) (layer "F.Cu") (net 5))
 (segment (start 111.75 88.25) (end 104.52 88.25) (width 0.25) (layer "F.Cu") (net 19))
 (segment (start 111.75 81.75) (end 111.75 88.25) (width 0.25) (layer "F.Cu") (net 19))
 (segment (start 104.52 88.25) (end 104 87.73) (width 0.25) (layer "F.Cu") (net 19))
 (segment (start 111.625 53.875) (end 104 61.5) (width 0.25) (layer "F.Cu") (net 6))
 (segment (start 122.685 53.875) (end 111.625 53.875) (width 0.25) (layer "F.Cu") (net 6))
 (segment (start 123.81 55) (end 122.685 53.875) (width 0.25) (layer "F.Cu") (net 6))
 (segment (start 123.81 95) (end 122.685 96.125) (width 0.25) (layer "F.Cu") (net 7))
 (segment (start 122.685 96.125) (end 114.125 96.125) (width 0.25) (layer "F.Cu") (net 7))
 (segment (start 103.175 63.595) (end 104 62.77) (width 0.25) (layer "F.Cu") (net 7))
 (segment (start 114.125 96.125) (end 107.5 89.5) (width 0.25) (layer "F.Cu") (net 7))
 (segment (start 103.175 68.675) (end 103.175 63.595) (width 0.25) (layer "F.Cu") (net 7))
 (segment (start 104.5 70) (end 103.175 68.675) (width 0.25) (layer "F.Cu") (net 7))
 (via (at 107.5 89.5) (size 0.8) (drill 0.4) (layers "F.Cu" "B.Cu") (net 7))
 (via (at 104.5 70) (size 0.8) (drill 0.4) (layers "F.Cu" "B.Cu") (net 7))
 (segment (start 107.5 89.5) (end 107.5 73) (width 0.25) (layer "B.Cu") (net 7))
 (segment (start 107.5 73) (end 104.5 70) (width 0.25) (layer "B.Cu") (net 7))
 (segment (start 188.81 55) (end 188.81 57.81) (width 0.25) (layer "F.Cu") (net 18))
 (segment (start 188.81 57.81) (end 195.5 64.5) (width 0.25) (layer "F.Cu") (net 18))
 (segment (start 188.81 72.46) (end 195.5 65.77) (width 0.25) (layer "F.Cu") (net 15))
 (segment (start 188.81 95) (end 188.81 72.46) (width 0.25) (layer "F.Cu") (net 15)))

